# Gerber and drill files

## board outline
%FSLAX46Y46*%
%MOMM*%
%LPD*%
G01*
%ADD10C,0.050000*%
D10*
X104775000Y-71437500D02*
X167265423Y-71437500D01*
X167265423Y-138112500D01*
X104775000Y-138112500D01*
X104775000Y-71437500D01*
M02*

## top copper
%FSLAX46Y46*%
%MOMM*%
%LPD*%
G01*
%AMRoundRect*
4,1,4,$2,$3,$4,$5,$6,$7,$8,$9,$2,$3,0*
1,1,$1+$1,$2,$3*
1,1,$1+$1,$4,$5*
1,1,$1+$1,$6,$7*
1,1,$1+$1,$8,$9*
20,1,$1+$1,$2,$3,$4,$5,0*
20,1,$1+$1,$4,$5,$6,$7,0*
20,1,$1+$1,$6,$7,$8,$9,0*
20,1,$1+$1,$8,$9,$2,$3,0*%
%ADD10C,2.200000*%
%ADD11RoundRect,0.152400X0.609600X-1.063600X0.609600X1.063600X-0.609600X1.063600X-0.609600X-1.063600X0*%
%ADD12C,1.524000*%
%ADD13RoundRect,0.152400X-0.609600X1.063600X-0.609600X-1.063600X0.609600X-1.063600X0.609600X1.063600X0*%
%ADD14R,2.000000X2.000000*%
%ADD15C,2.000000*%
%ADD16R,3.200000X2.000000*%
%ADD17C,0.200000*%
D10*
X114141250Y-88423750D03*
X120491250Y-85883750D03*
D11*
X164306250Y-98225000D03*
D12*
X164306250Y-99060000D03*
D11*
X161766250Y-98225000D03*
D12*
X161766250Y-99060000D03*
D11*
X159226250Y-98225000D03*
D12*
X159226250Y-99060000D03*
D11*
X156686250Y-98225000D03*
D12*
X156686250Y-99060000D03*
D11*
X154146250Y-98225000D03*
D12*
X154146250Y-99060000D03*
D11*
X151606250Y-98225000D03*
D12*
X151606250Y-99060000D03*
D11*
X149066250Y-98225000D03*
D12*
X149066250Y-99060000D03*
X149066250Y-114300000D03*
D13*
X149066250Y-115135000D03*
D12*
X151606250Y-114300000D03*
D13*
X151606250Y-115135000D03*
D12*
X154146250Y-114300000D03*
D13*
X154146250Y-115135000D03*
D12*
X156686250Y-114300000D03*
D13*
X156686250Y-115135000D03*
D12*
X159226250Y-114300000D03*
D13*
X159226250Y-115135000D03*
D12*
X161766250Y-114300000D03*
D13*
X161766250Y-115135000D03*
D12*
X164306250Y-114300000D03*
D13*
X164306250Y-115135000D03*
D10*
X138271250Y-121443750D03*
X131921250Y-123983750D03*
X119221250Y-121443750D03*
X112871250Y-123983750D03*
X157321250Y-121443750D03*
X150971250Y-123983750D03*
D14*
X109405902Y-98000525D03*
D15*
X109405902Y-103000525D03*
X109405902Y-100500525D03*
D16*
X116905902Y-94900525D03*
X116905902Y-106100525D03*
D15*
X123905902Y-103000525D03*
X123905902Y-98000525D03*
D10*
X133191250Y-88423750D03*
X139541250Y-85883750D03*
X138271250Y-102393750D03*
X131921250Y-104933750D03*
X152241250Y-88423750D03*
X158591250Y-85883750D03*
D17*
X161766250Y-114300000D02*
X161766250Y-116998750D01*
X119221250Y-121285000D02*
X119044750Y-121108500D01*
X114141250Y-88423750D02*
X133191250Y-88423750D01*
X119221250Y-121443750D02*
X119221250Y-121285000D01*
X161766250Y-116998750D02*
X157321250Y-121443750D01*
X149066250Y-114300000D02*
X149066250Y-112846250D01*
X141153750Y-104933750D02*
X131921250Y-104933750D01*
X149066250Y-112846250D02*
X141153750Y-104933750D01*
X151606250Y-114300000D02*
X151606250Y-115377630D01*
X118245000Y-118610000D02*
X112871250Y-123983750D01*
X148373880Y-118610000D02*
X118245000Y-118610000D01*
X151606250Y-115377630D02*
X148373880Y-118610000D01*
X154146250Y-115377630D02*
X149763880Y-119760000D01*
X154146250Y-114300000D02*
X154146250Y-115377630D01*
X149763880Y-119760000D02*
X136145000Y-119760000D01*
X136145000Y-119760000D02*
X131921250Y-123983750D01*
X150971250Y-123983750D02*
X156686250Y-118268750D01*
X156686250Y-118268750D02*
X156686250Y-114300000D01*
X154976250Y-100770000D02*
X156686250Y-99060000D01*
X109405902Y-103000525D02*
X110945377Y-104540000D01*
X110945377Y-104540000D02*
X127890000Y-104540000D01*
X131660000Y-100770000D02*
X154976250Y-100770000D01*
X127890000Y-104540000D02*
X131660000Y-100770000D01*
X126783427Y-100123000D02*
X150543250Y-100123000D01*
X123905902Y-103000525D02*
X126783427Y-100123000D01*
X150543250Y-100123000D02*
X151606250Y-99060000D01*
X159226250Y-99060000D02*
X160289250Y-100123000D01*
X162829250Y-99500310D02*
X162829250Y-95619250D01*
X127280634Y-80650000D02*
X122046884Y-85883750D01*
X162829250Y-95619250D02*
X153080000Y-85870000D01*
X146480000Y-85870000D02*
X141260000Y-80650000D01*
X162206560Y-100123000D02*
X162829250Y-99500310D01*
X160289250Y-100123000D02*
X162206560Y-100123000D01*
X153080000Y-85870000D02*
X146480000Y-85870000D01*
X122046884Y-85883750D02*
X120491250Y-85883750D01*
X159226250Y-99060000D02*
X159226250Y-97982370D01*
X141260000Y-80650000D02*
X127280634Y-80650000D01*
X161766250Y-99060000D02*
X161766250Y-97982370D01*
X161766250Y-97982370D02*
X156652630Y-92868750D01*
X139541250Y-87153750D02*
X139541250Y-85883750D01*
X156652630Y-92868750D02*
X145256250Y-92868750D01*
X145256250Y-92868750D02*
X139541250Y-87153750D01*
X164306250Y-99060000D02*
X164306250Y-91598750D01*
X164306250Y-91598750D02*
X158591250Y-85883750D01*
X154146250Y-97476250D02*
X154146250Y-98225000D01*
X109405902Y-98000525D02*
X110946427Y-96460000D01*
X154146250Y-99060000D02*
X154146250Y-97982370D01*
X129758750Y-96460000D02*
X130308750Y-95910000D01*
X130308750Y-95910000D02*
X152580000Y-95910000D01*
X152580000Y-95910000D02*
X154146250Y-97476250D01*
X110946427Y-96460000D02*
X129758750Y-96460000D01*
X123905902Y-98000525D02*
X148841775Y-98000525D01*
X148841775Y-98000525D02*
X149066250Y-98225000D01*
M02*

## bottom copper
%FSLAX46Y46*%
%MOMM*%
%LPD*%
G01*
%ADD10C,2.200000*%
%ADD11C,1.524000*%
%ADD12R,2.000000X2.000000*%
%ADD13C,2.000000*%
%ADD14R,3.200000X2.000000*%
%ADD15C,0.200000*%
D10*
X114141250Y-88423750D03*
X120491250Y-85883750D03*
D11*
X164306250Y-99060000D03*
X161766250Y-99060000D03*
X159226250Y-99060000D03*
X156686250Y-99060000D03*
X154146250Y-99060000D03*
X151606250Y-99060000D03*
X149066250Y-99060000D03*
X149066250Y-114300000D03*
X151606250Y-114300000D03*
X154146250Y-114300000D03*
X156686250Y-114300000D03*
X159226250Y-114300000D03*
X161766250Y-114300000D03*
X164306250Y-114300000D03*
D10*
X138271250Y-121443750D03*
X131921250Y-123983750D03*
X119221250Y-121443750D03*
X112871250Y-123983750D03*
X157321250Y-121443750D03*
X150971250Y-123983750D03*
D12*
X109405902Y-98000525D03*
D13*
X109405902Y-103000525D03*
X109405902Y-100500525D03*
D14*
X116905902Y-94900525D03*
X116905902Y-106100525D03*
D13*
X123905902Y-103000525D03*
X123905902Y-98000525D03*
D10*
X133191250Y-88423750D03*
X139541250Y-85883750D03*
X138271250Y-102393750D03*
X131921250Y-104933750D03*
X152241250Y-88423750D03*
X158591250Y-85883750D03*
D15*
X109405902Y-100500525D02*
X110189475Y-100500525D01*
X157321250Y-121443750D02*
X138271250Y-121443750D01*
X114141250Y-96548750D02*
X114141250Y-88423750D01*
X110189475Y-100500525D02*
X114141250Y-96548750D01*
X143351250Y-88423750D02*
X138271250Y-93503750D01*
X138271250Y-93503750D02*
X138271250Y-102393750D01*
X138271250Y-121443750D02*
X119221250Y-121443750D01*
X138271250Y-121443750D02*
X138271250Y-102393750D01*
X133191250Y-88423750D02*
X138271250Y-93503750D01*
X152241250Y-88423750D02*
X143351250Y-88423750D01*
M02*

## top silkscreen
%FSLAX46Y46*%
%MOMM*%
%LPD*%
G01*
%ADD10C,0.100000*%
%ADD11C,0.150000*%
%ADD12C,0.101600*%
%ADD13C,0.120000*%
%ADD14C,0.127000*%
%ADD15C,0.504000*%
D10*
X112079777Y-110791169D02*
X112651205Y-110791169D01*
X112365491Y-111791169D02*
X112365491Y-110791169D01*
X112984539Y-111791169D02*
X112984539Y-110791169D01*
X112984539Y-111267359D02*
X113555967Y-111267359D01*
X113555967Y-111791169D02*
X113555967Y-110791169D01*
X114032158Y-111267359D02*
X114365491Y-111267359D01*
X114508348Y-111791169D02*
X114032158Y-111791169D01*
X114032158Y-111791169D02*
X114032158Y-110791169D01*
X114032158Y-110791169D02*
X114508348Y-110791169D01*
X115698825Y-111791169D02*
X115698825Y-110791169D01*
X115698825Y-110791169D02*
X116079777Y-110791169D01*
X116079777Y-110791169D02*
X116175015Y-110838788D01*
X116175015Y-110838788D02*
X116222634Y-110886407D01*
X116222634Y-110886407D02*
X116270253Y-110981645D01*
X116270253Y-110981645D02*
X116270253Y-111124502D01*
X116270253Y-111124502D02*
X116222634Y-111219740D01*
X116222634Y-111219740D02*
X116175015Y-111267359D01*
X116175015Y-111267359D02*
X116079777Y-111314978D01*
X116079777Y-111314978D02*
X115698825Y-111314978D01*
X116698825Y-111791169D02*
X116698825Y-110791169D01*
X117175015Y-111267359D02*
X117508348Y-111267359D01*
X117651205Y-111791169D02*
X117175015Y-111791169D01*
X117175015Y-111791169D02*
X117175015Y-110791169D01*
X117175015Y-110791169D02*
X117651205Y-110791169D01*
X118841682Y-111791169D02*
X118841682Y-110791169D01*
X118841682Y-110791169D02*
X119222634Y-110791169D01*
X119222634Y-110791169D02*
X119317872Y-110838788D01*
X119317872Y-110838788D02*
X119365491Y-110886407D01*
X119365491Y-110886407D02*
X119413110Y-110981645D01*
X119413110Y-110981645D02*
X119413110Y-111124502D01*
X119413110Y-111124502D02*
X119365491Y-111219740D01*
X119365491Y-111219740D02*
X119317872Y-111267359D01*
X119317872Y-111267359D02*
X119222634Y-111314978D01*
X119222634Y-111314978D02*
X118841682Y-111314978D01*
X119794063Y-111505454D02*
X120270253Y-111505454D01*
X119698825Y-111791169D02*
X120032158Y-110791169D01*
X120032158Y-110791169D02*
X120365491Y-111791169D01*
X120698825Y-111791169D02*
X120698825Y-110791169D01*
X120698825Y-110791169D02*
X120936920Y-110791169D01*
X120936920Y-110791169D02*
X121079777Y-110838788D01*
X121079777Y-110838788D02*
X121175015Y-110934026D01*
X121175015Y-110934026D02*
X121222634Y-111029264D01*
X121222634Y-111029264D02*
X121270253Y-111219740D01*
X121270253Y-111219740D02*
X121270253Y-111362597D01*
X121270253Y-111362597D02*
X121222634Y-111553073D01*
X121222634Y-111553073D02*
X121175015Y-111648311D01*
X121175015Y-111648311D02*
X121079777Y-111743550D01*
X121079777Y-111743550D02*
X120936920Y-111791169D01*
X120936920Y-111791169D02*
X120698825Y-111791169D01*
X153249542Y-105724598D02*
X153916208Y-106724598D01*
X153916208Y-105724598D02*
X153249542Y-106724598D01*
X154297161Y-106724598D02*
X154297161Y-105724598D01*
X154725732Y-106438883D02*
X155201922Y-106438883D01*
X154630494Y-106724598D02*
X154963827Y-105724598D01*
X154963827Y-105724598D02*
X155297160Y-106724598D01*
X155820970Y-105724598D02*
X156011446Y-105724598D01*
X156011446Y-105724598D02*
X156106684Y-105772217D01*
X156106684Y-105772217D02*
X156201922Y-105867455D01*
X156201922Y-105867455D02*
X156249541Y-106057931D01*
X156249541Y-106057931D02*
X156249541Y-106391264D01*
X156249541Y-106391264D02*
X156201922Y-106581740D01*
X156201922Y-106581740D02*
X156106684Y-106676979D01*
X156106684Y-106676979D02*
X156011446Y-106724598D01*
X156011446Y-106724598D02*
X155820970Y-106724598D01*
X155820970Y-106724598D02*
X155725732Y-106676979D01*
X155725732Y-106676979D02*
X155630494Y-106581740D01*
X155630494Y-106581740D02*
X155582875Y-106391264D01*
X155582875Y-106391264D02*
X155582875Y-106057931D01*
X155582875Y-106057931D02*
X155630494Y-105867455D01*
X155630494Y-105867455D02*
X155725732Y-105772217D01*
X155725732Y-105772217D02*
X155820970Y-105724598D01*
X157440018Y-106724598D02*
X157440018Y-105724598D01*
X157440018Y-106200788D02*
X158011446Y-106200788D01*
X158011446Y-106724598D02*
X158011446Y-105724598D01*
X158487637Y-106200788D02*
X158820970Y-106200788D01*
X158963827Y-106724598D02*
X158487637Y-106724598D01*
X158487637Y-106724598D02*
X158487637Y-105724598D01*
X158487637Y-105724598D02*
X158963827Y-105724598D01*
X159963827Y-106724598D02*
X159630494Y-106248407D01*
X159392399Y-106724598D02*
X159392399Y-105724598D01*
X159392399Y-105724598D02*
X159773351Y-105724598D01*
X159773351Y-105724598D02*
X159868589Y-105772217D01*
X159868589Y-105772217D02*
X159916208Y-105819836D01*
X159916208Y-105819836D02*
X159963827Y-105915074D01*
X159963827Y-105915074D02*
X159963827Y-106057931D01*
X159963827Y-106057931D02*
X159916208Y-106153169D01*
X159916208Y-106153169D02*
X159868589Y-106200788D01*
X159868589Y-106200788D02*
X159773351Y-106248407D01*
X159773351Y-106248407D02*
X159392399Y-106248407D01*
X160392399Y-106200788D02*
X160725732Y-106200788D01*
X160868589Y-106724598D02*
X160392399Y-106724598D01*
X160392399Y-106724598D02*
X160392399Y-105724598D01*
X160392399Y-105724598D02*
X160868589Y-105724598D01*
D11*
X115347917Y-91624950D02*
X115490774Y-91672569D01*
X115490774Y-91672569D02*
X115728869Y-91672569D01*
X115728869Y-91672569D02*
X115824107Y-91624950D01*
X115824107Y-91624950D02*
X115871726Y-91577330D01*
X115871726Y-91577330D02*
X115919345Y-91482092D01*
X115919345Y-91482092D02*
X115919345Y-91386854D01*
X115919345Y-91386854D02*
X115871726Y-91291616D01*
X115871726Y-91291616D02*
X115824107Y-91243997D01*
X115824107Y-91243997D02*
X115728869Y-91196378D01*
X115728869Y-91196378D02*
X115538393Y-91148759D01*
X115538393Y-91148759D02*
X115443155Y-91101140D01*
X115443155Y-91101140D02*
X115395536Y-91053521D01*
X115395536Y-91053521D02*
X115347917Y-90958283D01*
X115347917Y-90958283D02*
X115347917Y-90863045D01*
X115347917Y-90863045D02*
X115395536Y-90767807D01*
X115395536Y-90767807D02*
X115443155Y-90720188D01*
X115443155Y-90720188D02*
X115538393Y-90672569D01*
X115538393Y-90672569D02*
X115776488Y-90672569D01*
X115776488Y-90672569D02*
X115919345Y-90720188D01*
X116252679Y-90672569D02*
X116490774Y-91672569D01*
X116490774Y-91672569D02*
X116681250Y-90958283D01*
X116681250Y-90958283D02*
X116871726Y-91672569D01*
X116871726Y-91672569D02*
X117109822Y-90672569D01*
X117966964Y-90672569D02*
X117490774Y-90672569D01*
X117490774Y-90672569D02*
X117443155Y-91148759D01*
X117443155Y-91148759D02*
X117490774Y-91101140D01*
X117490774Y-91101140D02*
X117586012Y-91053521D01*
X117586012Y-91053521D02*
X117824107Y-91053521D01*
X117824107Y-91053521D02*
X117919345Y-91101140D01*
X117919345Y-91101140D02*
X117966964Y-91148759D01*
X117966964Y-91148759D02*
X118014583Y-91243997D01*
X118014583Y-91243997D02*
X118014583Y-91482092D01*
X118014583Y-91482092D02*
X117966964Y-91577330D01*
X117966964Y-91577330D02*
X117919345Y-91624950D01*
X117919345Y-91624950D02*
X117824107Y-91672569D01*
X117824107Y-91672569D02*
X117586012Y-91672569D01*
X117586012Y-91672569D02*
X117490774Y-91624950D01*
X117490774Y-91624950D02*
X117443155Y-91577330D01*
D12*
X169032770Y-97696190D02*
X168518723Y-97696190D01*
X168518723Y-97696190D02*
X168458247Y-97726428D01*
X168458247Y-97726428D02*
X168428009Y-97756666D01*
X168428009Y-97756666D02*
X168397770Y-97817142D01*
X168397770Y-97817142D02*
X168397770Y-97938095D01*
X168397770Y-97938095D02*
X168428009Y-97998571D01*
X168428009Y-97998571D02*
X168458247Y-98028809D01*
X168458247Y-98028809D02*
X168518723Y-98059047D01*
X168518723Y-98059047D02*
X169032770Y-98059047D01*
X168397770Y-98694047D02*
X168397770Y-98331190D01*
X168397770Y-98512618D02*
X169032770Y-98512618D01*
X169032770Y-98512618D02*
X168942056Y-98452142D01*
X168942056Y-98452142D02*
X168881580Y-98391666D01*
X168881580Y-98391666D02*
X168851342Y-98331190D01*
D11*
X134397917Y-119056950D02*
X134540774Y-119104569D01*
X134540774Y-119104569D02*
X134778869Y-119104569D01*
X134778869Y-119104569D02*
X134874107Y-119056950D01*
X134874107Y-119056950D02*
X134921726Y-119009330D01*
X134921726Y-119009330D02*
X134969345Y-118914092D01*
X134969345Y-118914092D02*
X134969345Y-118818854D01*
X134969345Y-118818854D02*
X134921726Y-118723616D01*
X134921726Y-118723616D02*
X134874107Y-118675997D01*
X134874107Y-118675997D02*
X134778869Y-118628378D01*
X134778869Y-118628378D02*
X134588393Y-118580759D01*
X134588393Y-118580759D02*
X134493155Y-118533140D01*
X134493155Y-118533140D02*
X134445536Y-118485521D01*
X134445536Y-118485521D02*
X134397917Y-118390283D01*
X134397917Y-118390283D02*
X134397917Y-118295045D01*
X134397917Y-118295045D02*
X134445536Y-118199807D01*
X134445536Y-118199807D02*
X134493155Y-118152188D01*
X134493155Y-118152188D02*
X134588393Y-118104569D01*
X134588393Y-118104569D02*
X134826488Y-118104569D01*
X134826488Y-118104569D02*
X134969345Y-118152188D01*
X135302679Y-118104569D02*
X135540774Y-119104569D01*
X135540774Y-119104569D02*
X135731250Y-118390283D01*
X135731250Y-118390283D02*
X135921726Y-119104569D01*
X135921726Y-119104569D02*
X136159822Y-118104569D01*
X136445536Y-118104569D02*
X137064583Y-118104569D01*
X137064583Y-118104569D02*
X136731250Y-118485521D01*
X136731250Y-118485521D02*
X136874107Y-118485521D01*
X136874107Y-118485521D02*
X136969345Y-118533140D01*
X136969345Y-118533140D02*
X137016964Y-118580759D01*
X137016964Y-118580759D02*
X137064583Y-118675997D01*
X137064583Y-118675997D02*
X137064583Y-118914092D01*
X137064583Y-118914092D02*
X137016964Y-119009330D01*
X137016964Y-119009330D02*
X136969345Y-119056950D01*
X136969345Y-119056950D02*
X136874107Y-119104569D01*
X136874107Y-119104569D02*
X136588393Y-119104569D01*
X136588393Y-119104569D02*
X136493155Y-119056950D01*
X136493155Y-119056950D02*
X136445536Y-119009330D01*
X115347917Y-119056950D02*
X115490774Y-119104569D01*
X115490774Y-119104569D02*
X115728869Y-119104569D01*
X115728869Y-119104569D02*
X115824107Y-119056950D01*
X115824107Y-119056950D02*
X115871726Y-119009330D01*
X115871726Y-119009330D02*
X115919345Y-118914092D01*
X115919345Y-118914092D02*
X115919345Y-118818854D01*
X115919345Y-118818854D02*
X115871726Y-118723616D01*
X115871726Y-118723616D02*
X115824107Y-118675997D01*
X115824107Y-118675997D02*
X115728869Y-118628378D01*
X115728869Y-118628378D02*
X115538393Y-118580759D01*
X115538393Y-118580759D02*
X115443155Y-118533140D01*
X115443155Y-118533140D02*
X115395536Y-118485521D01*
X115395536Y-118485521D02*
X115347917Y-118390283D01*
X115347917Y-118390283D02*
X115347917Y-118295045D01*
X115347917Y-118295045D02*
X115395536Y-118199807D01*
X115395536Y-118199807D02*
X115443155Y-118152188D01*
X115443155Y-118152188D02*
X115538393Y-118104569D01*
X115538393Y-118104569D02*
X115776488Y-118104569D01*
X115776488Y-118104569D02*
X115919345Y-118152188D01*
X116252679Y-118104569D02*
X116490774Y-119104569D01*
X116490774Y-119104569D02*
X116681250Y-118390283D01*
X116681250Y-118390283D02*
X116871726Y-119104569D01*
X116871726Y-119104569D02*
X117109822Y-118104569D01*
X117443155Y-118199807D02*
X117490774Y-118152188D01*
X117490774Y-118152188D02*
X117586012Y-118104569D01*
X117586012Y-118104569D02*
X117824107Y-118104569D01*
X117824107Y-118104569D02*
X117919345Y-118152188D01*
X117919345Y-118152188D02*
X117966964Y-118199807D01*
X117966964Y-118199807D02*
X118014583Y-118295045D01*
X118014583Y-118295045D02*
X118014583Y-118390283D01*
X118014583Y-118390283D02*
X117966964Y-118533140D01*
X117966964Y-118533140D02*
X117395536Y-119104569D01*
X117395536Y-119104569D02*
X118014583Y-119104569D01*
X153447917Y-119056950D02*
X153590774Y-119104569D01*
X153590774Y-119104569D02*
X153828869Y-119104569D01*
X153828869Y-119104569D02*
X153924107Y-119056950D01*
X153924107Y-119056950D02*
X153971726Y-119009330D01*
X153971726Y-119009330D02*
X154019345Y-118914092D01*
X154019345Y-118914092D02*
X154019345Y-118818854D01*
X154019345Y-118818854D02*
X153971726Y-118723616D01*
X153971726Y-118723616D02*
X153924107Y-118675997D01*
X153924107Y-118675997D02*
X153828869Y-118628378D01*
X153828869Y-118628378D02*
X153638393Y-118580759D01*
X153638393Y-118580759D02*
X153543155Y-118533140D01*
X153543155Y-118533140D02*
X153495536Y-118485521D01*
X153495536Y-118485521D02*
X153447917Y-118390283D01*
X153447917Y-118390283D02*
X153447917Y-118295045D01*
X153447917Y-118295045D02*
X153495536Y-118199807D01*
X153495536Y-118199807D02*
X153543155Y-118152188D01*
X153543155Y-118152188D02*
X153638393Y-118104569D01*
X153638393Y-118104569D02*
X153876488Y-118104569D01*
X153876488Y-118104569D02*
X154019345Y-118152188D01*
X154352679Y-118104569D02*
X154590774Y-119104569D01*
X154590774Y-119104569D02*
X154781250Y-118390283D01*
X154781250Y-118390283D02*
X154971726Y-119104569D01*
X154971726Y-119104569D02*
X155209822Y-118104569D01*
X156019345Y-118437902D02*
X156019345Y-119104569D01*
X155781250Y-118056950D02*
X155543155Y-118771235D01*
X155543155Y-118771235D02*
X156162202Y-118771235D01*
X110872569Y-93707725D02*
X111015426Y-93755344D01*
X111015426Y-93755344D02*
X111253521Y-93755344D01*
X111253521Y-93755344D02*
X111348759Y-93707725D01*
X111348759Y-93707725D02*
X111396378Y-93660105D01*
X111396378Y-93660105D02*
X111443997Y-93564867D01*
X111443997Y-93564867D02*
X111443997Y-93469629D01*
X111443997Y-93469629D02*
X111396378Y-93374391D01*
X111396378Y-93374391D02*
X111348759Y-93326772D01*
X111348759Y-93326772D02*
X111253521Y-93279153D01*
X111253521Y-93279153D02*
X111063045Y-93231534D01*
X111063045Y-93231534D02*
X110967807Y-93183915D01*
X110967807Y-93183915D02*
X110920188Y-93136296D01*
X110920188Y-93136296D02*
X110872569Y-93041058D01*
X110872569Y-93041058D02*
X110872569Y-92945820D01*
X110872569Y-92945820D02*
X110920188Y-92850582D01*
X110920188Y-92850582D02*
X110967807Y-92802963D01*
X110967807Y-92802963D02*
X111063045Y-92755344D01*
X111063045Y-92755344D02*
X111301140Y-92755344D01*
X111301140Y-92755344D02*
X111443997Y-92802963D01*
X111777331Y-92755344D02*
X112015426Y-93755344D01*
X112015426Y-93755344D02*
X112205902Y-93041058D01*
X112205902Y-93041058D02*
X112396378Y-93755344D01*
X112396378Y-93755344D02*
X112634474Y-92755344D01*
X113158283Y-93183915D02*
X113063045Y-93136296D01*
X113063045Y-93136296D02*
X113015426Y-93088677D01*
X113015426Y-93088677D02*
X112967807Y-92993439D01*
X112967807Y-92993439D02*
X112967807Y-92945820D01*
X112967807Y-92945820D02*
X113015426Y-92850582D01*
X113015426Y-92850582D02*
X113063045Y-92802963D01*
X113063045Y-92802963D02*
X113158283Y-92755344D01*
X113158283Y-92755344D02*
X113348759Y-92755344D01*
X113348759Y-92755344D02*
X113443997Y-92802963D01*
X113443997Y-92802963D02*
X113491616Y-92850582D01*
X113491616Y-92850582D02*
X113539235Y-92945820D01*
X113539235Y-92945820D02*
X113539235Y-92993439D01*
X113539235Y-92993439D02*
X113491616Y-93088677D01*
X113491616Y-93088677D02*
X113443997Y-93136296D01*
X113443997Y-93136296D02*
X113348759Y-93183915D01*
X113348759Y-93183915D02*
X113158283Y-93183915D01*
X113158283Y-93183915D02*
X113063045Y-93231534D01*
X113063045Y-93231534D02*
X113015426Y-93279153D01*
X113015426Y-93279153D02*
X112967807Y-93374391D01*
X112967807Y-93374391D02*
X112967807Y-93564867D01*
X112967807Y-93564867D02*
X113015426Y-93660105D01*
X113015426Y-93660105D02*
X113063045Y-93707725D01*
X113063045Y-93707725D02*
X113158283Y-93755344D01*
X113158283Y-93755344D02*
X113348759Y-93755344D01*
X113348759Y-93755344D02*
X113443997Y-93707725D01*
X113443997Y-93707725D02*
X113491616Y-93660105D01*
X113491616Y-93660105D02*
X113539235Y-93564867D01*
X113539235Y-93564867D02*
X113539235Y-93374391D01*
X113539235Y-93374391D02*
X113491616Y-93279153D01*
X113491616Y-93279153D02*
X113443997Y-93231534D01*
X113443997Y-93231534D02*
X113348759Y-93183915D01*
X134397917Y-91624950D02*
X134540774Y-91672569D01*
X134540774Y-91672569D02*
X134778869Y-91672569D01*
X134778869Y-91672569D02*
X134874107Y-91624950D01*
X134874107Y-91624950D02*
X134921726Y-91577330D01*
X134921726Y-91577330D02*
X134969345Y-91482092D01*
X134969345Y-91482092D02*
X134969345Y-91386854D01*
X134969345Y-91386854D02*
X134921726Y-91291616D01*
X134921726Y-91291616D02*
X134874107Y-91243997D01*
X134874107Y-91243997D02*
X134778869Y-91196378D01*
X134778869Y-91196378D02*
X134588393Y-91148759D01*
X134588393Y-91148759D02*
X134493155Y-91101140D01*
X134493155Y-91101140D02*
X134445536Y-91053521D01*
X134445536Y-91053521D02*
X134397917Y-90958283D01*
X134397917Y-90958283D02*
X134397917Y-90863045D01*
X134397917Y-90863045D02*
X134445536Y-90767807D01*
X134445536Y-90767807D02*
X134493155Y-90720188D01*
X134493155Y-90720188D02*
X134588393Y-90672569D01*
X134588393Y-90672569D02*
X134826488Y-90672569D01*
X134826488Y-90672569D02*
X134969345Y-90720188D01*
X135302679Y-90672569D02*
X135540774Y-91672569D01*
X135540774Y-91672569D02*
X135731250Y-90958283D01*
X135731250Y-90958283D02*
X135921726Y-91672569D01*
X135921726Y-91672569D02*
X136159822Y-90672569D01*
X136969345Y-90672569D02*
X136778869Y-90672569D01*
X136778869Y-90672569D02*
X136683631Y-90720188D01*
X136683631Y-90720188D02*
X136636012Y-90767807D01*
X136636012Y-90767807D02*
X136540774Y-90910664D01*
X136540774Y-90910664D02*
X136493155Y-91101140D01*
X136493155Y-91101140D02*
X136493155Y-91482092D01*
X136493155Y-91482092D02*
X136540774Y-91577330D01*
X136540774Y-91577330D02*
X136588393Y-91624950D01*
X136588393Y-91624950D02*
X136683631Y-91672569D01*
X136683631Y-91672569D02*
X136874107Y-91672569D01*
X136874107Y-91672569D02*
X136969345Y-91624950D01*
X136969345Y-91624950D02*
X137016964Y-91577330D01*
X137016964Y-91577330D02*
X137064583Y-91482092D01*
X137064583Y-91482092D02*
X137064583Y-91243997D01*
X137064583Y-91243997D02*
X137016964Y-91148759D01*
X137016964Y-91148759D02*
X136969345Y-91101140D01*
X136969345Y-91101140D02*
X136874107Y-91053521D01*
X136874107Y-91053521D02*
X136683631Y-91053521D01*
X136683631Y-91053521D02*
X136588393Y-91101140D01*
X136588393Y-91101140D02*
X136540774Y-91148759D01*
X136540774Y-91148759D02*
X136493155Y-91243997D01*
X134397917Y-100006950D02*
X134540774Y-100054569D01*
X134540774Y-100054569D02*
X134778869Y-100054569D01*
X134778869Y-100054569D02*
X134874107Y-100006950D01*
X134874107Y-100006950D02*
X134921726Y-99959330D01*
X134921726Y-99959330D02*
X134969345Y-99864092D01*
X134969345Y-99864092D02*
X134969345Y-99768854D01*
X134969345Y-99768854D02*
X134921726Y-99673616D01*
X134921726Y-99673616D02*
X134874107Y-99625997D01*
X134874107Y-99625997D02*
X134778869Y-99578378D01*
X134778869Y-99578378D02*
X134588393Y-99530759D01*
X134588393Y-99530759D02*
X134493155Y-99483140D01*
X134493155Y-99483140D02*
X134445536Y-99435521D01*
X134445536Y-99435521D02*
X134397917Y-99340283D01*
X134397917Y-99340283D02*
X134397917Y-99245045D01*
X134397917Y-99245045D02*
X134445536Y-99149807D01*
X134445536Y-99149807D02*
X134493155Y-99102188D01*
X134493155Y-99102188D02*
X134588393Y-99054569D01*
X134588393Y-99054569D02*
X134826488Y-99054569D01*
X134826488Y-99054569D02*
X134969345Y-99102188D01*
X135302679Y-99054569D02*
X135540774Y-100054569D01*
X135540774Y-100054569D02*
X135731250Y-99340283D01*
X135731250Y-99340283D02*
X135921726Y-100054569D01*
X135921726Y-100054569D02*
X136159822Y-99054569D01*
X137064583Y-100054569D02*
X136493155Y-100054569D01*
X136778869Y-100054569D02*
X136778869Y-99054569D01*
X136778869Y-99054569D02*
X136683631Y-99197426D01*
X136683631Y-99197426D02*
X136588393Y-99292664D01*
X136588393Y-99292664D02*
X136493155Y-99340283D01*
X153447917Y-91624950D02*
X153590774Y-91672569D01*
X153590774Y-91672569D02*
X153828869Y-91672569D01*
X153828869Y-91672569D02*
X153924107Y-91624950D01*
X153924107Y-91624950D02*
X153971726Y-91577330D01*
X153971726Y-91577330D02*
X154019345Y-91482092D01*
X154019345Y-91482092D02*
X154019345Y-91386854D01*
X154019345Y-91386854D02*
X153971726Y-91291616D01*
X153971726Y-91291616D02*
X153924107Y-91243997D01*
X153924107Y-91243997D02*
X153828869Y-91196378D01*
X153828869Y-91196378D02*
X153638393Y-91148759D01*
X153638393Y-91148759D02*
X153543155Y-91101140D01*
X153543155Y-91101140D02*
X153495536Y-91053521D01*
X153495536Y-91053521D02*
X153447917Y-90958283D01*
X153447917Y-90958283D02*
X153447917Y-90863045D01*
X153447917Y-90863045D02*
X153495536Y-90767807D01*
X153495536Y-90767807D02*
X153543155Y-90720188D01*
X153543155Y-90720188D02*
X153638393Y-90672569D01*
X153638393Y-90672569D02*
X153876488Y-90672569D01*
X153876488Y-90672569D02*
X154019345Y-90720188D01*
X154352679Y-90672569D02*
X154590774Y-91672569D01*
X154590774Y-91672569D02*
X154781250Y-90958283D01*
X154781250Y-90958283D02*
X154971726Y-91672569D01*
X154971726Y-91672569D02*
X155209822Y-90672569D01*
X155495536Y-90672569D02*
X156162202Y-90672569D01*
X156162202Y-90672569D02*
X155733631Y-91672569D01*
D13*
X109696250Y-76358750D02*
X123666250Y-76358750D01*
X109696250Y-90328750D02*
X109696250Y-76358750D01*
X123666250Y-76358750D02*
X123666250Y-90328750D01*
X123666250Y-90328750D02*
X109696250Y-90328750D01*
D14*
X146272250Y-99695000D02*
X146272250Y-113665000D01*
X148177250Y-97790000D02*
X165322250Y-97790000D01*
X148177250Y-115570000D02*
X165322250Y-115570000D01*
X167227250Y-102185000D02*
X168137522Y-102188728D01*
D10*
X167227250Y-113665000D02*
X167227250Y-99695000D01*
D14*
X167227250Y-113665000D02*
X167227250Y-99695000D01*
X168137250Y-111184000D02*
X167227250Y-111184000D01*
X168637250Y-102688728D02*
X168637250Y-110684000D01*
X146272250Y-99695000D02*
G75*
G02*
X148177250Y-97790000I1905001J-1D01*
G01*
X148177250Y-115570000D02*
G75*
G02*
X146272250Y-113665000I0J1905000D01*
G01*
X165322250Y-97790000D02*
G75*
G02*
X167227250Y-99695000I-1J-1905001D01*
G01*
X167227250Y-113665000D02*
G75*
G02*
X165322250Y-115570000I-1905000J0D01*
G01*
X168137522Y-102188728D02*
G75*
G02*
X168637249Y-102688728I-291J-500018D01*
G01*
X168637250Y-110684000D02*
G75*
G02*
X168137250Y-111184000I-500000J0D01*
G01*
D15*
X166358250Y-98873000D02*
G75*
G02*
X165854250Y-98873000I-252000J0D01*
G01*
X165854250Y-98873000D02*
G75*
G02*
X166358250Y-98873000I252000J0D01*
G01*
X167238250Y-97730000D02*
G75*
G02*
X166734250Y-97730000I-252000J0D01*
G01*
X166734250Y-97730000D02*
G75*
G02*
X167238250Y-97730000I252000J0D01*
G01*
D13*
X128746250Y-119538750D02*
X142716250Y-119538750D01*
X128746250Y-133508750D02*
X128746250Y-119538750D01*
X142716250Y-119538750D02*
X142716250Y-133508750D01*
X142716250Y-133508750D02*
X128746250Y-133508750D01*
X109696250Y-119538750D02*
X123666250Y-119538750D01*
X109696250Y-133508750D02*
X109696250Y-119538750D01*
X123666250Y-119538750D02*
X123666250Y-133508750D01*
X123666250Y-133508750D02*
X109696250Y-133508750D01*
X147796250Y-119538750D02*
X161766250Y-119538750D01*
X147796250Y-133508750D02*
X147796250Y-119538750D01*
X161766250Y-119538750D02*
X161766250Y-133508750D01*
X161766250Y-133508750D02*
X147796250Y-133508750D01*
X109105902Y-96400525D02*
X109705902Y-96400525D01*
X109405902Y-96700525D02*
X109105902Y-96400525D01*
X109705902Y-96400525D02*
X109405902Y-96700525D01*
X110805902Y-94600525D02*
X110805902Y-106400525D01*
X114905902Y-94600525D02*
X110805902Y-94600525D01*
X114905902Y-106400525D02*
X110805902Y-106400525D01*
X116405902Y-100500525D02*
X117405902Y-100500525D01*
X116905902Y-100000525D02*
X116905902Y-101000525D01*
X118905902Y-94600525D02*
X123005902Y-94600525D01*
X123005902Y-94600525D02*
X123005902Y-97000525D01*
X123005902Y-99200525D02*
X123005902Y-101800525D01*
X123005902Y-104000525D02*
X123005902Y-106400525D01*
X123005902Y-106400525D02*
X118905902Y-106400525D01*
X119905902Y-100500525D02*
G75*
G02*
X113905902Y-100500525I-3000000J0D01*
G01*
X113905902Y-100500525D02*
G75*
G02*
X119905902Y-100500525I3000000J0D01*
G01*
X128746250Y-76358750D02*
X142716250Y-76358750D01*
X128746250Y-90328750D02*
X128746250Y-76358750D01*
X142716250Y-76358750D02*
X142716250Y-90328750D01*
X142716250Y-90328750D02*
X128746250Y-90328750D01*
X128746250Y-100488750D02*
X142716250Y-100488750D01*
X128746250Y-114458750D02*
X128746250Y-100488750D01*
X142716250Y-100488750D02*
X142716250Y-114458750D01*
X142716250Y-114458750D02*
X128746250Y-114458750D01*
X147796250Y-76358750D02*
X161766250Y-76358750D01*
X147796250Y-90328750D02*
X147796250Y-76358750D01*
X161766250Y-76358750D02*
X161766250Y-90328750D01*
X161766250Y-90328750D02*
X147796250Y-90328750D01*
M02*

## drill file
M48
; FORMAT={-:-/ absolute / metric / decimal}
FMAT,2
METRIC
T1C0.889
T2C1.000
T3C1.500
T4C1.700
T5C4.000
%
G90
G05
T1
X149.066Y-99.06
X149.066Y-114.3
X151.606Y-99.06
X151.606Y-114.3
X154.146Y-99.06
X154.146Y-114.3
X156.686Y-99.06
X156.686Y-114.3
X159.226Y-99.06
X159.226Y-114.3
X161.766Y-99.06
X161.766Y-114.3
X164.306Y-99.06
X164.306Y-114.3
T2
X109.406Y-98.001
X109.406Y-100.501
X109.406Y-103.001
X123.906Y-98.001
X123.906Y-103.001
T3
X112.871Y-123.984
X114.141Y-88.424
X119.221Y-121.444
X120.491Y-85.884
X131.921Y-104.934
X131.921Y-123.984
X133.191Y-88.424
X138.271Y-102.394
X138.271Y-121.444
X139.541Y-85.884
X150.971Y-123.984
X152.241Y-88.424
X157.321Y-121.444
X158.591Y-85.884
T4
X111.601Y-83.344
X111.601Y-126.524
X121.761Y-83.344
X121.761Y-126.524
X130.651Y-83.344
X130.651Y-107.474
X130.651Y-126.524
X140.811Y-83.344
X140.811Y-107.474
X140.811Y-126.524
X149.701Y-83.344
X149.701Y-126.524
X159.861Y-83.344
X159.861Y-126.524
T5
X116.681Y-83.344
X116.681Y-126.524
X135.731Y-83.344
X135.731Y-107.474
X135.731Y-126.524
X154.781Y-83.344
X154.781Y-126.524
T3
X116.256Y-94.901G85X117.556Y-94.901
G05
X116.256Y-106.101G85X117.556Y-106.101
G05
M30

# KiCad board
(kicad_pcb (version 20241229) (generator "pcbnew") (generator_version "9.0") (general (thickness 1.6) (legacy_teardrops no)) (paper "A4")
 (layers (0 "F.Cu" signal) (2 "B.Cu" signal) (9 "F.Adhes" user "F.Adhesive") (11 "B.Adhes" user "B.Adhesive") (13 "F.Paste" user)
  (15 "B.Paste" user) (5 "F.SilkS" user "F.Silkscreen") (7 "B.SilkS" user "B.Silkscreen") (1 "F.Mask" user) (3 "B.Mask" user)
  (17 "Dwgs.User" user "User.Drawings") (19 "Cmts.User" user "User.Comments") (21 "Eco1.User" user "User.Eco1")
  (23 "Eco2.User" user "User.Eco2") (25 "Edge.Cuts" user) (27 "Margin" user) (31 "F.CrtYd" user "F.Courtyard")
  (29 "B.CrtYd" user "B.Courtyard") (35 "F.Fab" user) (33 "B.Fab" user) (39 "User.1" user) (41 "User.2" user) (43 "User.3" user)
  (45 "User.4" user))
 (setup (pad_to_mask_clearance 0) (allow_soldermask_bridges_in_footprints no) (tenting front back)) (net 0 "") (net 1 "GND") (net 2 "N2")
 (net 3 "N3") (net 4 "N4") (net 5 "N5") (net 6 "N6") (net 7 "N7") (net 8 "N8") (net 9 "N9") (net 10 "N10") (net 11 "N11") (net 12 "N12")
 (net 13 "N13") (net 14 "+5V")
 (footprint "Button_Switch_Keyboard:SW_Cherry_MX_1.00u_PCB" (layer "F.Cu") (at 114.14125 88.42375 180)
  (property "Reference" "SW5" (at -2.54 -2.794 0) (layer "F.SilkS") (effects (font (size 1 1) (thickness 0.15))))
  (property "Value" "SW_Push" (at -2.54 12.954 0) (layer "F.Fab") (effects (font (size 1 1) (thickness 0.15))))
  (fp_line (start 4.445 12.065) (end -9.525 12.065) (stroke (width 0.12) (type solid)) (layer "F.SilkS"))
  (fp_line (start 4.445 -1.905) (end 4.445 12.065) (stroke (width 0.12) (type solid)) (layer "F.SilkS"))
  (fp_line (start -9.525 12.065) (end -9.525 -1.905) (stroke (width 0.12) (type solid)) (layer "F.SilkS"))
  (fp_line (start -9.525 -1.905) (end 4.445 -1.905) (stroke (width 0.12) (type solid)) (layer "F.SilkS"))
  (pad "" np_thru_hole circle (at -7.62 5.08 180) (size 1.7 1.7) (drill 1.7) (layers "*.Cu" "*.Mask"))
  (pad "" np_thru_hole circle (at -2.54 5.08 180) (size 4 4) (drill 4) (layers "*.Cu" "*.Mask"))
  (pad "" np_thru_hole circle (at 2.54 5.08 180) (size 1.7 1.7) (drill 1.7) (layers "*.Cu" "*.Mask"))
  (pad "1" thru_hole circle (at 0 0 180) (size 2.2 2.2) (drill 1.5) (layers "*.Cu" "*.Mask") (remove_unused_layers no) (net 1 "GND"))
  (pad "2" thru_hole circle (at -6.35 2.54 180) (size 2.2 2.2) (drill 1.5) (layers "*.Cu" "*.Mask") (remove_unused_layers no) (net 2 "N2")))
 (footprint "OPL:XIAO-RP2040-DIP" (layer "F.Cu") (at 156.68625 106.68 -90)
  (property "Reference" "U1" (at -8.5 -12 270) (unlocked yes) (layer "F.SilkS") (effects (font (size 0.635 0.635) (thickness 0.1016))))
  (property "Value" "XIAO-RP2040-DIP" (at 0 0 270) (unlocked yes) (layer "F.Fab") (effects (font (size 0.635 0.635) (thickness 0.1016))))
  (fp_line (start -6.985 10.414) (end 6.985 10.414) (stroke (width 0.127) (type solid)) (layer "F.SilkS"))
  (fp_line (start -8.89 8.509) (end -8.89 -8.636) (stroke (width 0.127) (type solid)) (layer "F.SilkS"))
  (fp_line (start 8.89 8.509) (end 8.89 -8.636) (stroke (width 0.127) (type solid)) (layer "F.SilkS"))
  (fp_line (start -4.495 -10.541) (end -4.491272 -11.451272) (stroke (width 0.127) (type solid)) (layer "F.SilkS"))
  (fp_line (start 6.985 -10.541) (end -6.985 -10.541) (stroke (width 0.1) (type solid)) (layer "F.SilkS"))
  (fp_line (start 6.985 -10.541) (end -6.985 -10.541) (stroke (width 0.127) (type solid)) (layer "F.SilkS"))
  (fp_line (start 4.504 -11.451) (end 4.504 -10.541) (stroke (width 0.127) (type solid)) (layer "F.SilkS"))
  (fp_line (start -3.991272 -11.951) (end 4.004 -11.951) (stroke (width 0.127) (type solid)) (layer "F.SilkS"))
  (fp_arc (start -6.985 10.414) (mid -8.332038 9.856038) (end -8.89 8.509) (stroke (width 0.127) (type solid)) (layer "F.SilkS"))
  (fp_arc (start 8.89 8.509) (mid 8.332038 9.856038) (end 6.985 10.414) (stroke (width 0.127) (type solid)) (layer "F.SilkS"))
  (fp_arc (start -8.89 -8.636) (mid -8.332038 -9.983038) (end -6.985 -10.541) (stroke (width 0.127) (type solid)) (layer "F.SilkS"))
  (fp_arc (start 6.985 -10.541) (mid 8.332038 -9.983038) (end 8.89 -8.636) (stroke (width 0.127) (type solid)) (layer "F.SilkS"))
  (fp_arc (start -4.491272 -11.451272) (mid -4.344728 -11.80464) (end -3.991272 -11.951) (stroke (width 0.127) (type default))
   (layer "F.SilkS"))
  (fp_arc (start 4.004 -11.951) (mid 4.357553 -11.804553) (end 4.504 -11.451) (stroke (width 0.127) (type default)) (layer "F.SilkS"))
  (fp_circle (center -7.807 -9.42) (end -7.807 -9.674) (stroke (width 0.5) (type solid)) (fill yes) (layer "F.SilkS"))
  (fp_circle (center -8.95 -10.3) (end -8.95 -10.554) (stroke (width 0.5) (type solid)) (fill yes) (layer "F.SilkS"))
  (pad "1" smd roundrect (at -8.455 -7.62 90) (size 2.432 1.524) (layers "F.Cu" "F.Mask") (roundrect_rratio 0.1) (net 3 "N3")
   (thermal_bridge_angle 45))
  (pad "1" thru_hole circle (at -7.62 -7.62 90) (size 1.524 1.524) (drill 0.889) (layers "*.Cu" "*.Mask") (remove_unused_layers no)
   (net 3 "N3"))
  (pad "2" smd roundrect (at -8.455 -5.08 90) (size 2.432 1.524) (layers "F.Cu" "F.Mask") (roundrect_rratio 0.1) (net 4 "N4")
   (thermal_bridge_angle 45))
  (pad "2" thru_hole circle (at -7.62 -5.08 90) (size 1.524 1.524) (drill 0.889) (layers "*.Cu" "*.Mask") (remove_unused_layers no)
   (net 4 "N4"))
  (pad "3" smd roundrect (at -8.455 -2.54 90) (size 2.432 1.524) (layers "F.Cu" "F.Mask") (roundrect_rratio 0.1) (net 2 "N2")
   (thermal_bridge_angle 45))
  (pad "3" thru_hole circle (at -7.62 -2.54 90) (size 1.524 1.524) (drill 0.889) (layers "*.Cu" "*.Mask") (remove_unused_layers no)
   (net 2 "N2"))
  (pad "4" smd roundrect (at -8.455 0 90) (size 2.432 1.524) (layers "F.Cu" "F.Mask") (roundrect_rratio 0.1) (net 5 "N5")
   (thermal_bridge_angle 45))
  (pad "4" thru_hole circle (at -7.62 0 90) (size 1.524 1.524) (drill 0.889) (layers "*.Cu" "*.Mask") (remove_unused_layers no) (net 5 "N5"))
  (pad "5" smd roundrect (at -8.455 2.54 90) (size 2.432 1.524) (layers "F.Cu" "F.Mask") (roundrect_rratio 0.1) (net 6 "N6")
   (thermal_bridge_angle 45))
  (pad "5" thru_hole circle (at -7.62 2.54 90) (size 1.524 1.524) (drill 0.889) (layers "*.Cu" "*.Mask") (remove_unused_layers no)
   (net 6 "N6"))
  (pad "6" smd roundrect (at -8.455 5.08 90) (size 2.432 1.524) (layers "F.Cu" "F.Mask") (roundrect_rratio 0.1) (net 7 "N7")
   (thermal_bridge_angle 45))
  (pad "6" thru_hole circle (at -7.62 5.08 90) (size 1.524 1.524) (drill 0.889) (layers "*.Cu" "*.Mask") (remove_unused_layers no)
   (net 7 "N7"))
  (pad "7" smd roundrect (at -8.455 7.62 90) (size 2.432 1.524) (layers "F.Cu" "F.Mask") (roundrect_rratio 0.1) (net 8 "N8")
   (thermal_bridge_angle 45))
  (pad "7" thru_hole circle (at -7.62 7.62 90) (size 1.524 1.524) (drill 0.889) (layers "*.Cu" "*.Mask") (remove_unused_layers no)
   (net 8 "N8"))
  (pad "8" thru_hole circle (at 7.62 7.62 270) (size 1.524 1.524) (drill 0.889) (layers "*.Cu" "*.Mask") (remove_unused_layers no)
   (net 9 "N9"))
  (pad "8" smd roundrect (at 8.455 7.62 270) (size 2.432 1.524) (layers "F.Cu" "F.Mask") (roundrect_rratio 0.1) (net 9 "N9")
   (thermal_bridge_angle 45))
  (pad "9" thru_hole circle (at 7.62 5.08 270) (size 1.524 1.524) (drill 0.889) (layers "*.Cu" "*.Mask") (remove_unused_layers no)
   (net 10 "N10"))
  (pad "9" smd roundrect (at 8.455 5.08 270) (size 2.432 1.524) (layers "F.Cu" "F.Mask") (roundrect_rratio 0.1) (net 10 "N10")
   (thermal_bridge_angle 45))
  (pad "10" thru_hole circle (at 7.62 2.54 270) (size 1.524 1.524) (drill 0.889) (layers "*.Cu" "*.Mask") (remove_unused_layers no)
   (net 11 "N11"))
  (pad "10" smd roundrect (at 8.455 2.54 270) (size 2.432 1.524) (layers "F.Cu" "F.Mask") (roundrect_rratio 0.1) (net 11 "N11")
   (thermal_bridge_angle 45))
  (pad "11" thru_hole circle (at 7.62 0 270) (size 1.524 1.524) (drill 0.889) (layers "*.Cu" "*.Mask") (remove_unused_layers no)
   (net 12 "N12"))
  (pad "11" smd roundrect (at 8.455 0 270) (size 2.432 1.524) (layers "F.Cu" "F.Mask") (roundrect_rratio 0.1) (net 12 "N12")
   (thermal_bridge_angle 45))
  (pad "12" thru_hole circle (at 7.62 -2.54 270) (size 1.524 1.524) (drill 0.889) (layers "*.Cu" "*.Mask") (remove_unused_layers no)
   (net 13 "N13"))
  (pad "12" smd roundrect (at 8.455 -2.54 270) (size 2.432 1.524) (layers "F.Cu" "F.Mask") (roundrect_rratio 0.1) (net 13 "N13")
   (thermal_bridge_angle 45))
  (pad "13" thru_hole circle (at 7.62 -5.08 270) (size 1.524 1.524) (drill 0.889) (layers "*.Cu" "*.Mask") (remove_unused_layers no)
   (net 1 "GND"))
  (pad "13" smd roundrect (at 8.455 -5.08 270) (size 2.432 1.524) (layers "F.Cu" "F.Mask") (roundrect_rratio 0.1) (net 1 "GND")
   (thermal_bridge_angle 45))
  (pad "14" thru_hole circle (at 7.62 -7.62 270) (size 1.524 1.524) (drill 0.889) (layers "*.Cu" "*.Mask") (remove_unused_layers no)
   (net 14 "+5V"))
  (pad "14" smd roundrect (at 8.455 -7.62 270) (size 2.432 1.524) (layers "F.Cu" "F.Mask") (roundrect_rratio 0.1) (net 14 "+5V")
   (thermal_bridge_angle 45)))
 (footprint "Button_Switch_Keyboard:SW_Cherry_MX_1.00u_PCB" (layer "F.Cu") (at 138.27125 121.44375)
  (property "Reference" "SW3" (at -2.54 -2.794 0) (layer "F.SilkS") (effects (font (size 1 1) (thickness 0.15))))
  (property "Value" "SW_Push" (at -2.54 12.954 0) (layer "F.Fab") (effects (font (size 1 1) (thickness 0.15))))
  (fp_line (start -9.525 -1.905) (end 4.445 -1.905) (stroke (width 0.12) (type solid)) (layer "F.SilkS"))
  (fp_line (start -9.525 12.065) (end -9.525 -1.905) (stroke (width 0.12) (type solid)) (layer "F.SilkS"))
  (fp_line (start 4.445 -1.905) (end 4.445 12.065) (stroke (width 0.12) (type solid)) (layer "F.SilkS"))
  (fp_line (start 4.445 12.065) (end -9.525 12.065) (stroke (width 0.12) (type solid)) (layer "F.SilkS"))
  (pad "" np_thru_hole circle (at -7.62 5.08) (size 1.7 1.7) (drill 1.7) (layers "*.Cu" "*.Mask"))
  (pad "" np_thru_hole circle (at -2.54 5.08) (size 4 4) (drill 4) (layers "*.Cu" "*.Mask"))
  (pad "" np_thru_hole circle (at 2.54 5.08) (size 1.7 1.7) (drill 1.7) (layers "*.Cu" "*.Mask"))
  (pad "1" thru_hole circle (at 0 0) (size 2.2 2.2) (drill 1.5) (layers "*.Cu" "*.Mask") (remove_unused_layers no) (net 1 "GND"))
  (pad "2" thru_hole circle (at -6.35 2.54) (size 2.2 2.2) (drill 1.5) (layers "*.Cu" "*.Mask") (remove_unused_layers no) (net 11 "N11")))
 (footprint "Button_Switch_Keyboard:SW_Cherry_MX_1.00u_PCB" (layer "F.Cu") (at 119.22125 121.44375)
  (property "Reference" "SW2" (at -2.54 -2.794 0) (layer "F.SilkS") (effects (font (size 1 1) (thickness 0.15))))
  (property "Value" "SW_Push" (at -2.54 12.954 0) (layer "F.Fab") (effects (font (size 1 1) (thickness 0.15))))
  (fp_line (start -9.525 -1.905) (end 4.445 -1.905) (stroke (width 0.12) (type solid)) (layer "F.SilkS"))
  (fp_line (start -9.525 12.065) (end -9.525 -1.905) (stroke (width 0.12) (type solid)) (layer "F.SilkS"))
  (fp_line (start 4.445 -1.905) (end 4.445 12.065) (stroke (width 0.12) (type solid)) (layer "F.SilkS"))
  (fp_line (start 4.445 12.065) (end -9.525 12.065) (stroke (width 0.12) (type solid)) (layer "F.SilkS"))
  (pad "" np_thru_hole circle (at -7.62 5.08) (size 1.7 1.7) (drill 1.7) (layers "*.Cu" "*.Mask"))
  (pad "" np_thru_hole circle (at -2.54 5.08) (size 4 4) (drill 4) (layers "*.Cu" "*.Mask"))
  (pad "" np_thru_hole circle (at 2.54 5.08) (size 1.7 1.7) (drill 1.7) (layers "*.Cu" "*.Mask"))
  (pad "1" thru_hole circle (at 0 0) (size 2.2 2.2) (drill 1.5) (layers "*.Cu" "*.Mask") (remove_unused_layers no) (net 1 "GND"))
  (pad "2" thru_hole circle (at -6.35 2.54) (size 2.2 2.2) (drill 1.5) (layers "*.Cu" "*.Mask") (remove_unused_layers no) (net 10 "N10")))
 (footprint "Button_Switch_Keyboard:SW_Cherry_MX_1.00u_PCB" (layer "F.Cu") (at 157.32125 121.44375)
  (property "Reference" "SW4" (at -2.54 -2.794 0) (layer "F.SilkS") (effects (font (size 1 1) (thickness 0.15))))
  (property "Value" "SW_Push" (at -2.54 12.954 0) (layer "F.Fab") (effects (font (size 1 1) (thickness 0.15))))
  (fp_line (start -9.525 -1.905) (end 4.445 -1.905) (stroke (width 0.12) (type solid)) (layer "F.SilkS"))
  (fp_line (start -9.525 12.065) (end -9.525 -1.905) (stroke (width 0.12) (type solid)) (layer "F.SilkS"))
  (fp_line (start 4.445 -1.905) (end 4.445 12.065) (stroke (width 0.12) (type solid)) (layer "F.SilkS"))
  (fp_line (start 4.445 12.065) (end -9.525 12.065) (stroke (width 0.12) (type solid)) (layer "F.SilkS"))
  (pad "" np_thru_hole circle (at -7.62 5.08) (size 1.7 1.7) (drill 1.7) (layers "*.Cu" "*.Mask"))
  (pad "" np_thru_hole circle (at -2.54 5.08) (size 4 4) (drill 4) (layers "*.Cu" "*.Mask"))
  (pad "" np_thru_hole circle (at 2.54 5.08) (size 1.7 1.7) (drill 1.7) (layers "*.Cu" "*.Mask"))
  (pad "1" thru_hole circle (at 0 0) (size 2.2 2.2) (drill 1.5) (layers "*.Cu" "*.Mask") (remove_unused_layers no) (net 1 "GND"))
  (pad "2" thru_hole circle (at -6.35 2.54) (size 2.2 2.2) (drill 1.5) (layers "*.Cu" "*.Mask") (remove_unused_layers no) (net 12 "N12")))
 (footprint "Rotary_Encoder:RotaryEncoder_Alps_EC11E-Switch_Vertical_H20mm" (layer "F.Cu") (at 109.405902 98.000525)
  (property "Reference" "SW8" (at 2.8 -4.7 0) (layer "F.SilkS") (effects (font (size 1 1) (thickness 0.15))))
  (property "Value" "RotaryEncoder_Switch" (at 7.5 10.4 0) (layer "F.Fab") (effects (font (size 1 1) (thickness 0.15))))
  (fp_line (start -0.3 -1.6) (end 0.3 -1.6) (stroke (width 0.12) (type solid)) (layer "F.SilkS"))
  (fp_line (start 0 -1.3) (end -0.3 -1.6) (stroke (width 0.12) (type solid)) (layer "F.SilkS"))
  (fp_line (start 0.3 -1.6) (end 0 -1.3) (stroke (width 0.12) (type solid)) (layer "F.SilkS"))
  (fp_line (start 1.4 -3.4) (end 1.4 8.4) (stroke (width 0.12) (type solid)) (layer "F.SilkS"))
  (fp_line (start 5.5 -3.4) (end 1.4 -3.4) (stroke (width 0.12) (type solid)) (layer "F.SilkS"))
  (fp_line (start 5.5 8.4) (end 1.4 8.4) (stroke (width 0.12) (type solid)) (layer "F.SilkS"))
  (fp_line (start 7 2.5) (end 8 2.5) (stroke (width 0.12) (type solid)) (layer "F.SilkS"))
  (fp_line (start 7.5 2) (end 7.5 3) (stroke (width 0.12) (type solid)) (layer "F.SilkS"))
  (fp_line (start 9.5 -3.4) (end 13.6 -3.4) (stroke (width 0.12) (type solid)) (layer "F.SilkS"))
  (fp_line (start 13.6 -3.4) (end 13.6 -1) (stroke (width 0.12) (type solid)) (layer "F.SilkS"))
  (fp_line (start 13.6 1.2) (end 13.6 3.8) (stroke (width 0.12) (type solid)) (layer "F.SilkS"))
  (fp_line (start 13.6 6) (end 13.6 8.4) (stroke (width 0.12) (type solid)) (layer "F.SilkS"))
  (fp_line (start 13.6 8.4) (end 9.5 8.4) (stroke (width 0.12) (type solid)) (layer "F.SilkS"))
  (fp_circle (center 7.5 2.5) (end 10.5 2.5) (stroke (width 0.12) (type solid)) (fill no) (layer "F.SilkS"))
  (pad "A" thru_hole rect (at 0 0) (size 2 2) (drill 1) (layers "*.Cu" "*.Mask") (remove_unused_layers no) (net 6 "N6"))
  (pad "B" thru_hole circle (at 0 5) (size 2 2) (drill 1) (layers "*.Cu" "*.Mask") (remove_unused_layers no) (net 5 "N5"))
  (pad "C" thru_hole circle (at 0 2.5) (size 2 2) (drill 1) (layers "*.Cu" "*.Mask") (remove_unused_layers no) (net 1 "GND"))
  (pad "MP" thru_hole rect (at 7.5 -3.1) (size 3.2 2) (drill oval 2.8 1.5) (layers "*.Cu" "*.Mask") (remove_unused_layers no))
  (pad "MP" thru_hole rect (at 7.5 8.1) (size 3.2 2) (drill oval 2.8 1.5) (layers "*.Cu" "*.Mask") (remove_unused_layers no))
  (pad "S1" thru_hole circle (at 14.5 5) (size 2 2) (drill 1) (layers "*.Cu" "*.Mask") (remove_unused_layers no) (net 7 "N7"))
  (pad "S2" thru_hole circle (at 14.5 0) (size 2 2) (drill 1) (layers "*.Cu" "*.Mask") (remove_unused_layers no) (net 8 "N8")))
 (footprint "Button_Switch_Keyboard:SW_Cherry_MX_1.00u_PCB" (layer "F.Cu") (at 133.19125 88.42375 180)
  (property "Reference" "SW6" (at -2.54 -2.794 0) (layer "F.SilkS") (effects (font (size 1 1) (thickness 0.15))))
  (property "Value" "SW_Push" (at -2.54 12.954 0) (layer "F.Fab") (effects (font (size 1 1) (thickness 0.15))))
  (fp_line (start 4.445 12.065) (end -9.525 12.065) (stroke (width 0.12) (type solid)) (layer "F.SilkS"))
  (fp_line (start 4.445 -1.905) (end 4.445 12.065) (stroke (width 0.12) (type solid)) (layer "F.SilkS"))
  (fp_line (start -9.525 12.065) (end -9.525 -1.905) (stroke (width 0.12) (type solid)) (layer "F.SilkS"))
  (fp_line (start -9.525 -1.905) (end 4.445 -1.905) (stroke (width 0.12) (type solid)) (layer "F.SilkS"))
  (pad "" np_thru_hole circle (at -7.62 5.08 180) (size 1.7 1.7) (drill 1.7) (layers "*.Cu" "*.Mask"))
  (pad "" np_thru_hole circle (at -2.54 5.08 180) (size 4 4) (drill 4) (layers "*.Cu" "*.Mask"))
  (pad "" np_thru_hole circle (at 2.54 5.08 180) (size 1.7 1.7) (drill 1.7) (layers "*.Cu" "*.Mask"))
  (pad "1" thru_hole circle (at 0 0 180) (size 2.2 2.2) (drill 1.5) (layers "*.Cu" "*.Mask") (remove_unused_layers no) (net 1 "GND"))
  (pad "2" thru_hole circle (at -6.35 2.54 180) (size 2.2 2.2) (drill 1.5) (layers "*.Cu" "*.Mask") (remove_unused_layers no) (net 4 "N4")))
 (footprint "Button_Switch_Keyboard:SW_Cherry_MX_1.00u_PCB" (layer "F.Cu") (at 138.27125 102.39375)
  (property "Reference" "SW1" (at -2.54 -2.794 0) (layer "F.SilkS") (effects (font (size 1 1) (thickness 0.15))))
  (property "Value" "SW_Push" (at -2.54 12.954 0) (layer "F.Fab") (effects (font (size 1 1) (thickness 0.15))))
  (fp_line (start -9.525 -1.905) (end 4.445 -1.905) (stroke (width 0.12) (type solid)) (layer "F.SilkS"))
  (fp_line (start -9.525 12.065) (end -9.525 -1.905) (stroke (width 0.12) (type solid)) (layer "F.SilkS"))
  (fp_line (start 4.445 -1.905) (end 4.445 12.065) (stroke (width 0.12) (type solid)) (layer "F.SilkS"))
  (fp_line (start 4.445 12.065) (end -9.525 12.065) (stroke (width 0.12) (type solid)) (layer "F.SilkS"))
  (pad "" np_thru_hole circle (at -7.62 5.08) (size 1.7 1.7) (drill 1.7) (layers "*.Cu" "*.Mask"))
  (pad "" np_thru_hole circle (at -2.54 5.08) (size 4 4) (drill 4) (layers "*.Cu" "*.Mask"))
  (pad "" np_thru_hole circle (at 2.54 5.08) (size 1.7 1.7) (drill 1.7) (layers "*.Cu" "*.Mask"))
  (pad "1" thru_hole circle (at 0 0) (size 2.2 2.2) (drill 1.5) (layers "*.Cu" "*.Mask") (remove_unused_layers no) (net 1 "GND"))
  (pad "2" thru_hole circle (at -6.35 2.54) (size 2.2 2.2) (drill 1.5) (layers "*.Cu" "*.Mask") (remove_unused_layers no) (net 9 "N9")))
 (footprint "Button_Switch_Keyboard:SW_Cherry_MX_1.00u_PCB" (layer "F.Cu") (at 152.24125 88.42375 180)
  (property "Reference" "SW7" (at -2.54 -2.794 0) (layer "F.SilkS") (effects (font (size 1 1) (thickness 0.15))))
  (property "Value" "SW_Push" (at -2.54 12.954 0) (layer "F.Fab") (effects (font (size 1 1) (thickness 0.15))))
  (fp_line (start 4.445 12.065) (end -9.525 12.065) (stroke (width 0.12) (type solid)) (layer "F.SilkS"))
  (fp_line (start 4.445 -1.905) (end 4.445 12.065) (stroke (width 0.12) (type solid)) (layer "F.SilkS"))
  (fp_line (start -9.525 12.065) (end -9.525 -1.905) (stroke (width 0.12) (type solid)) (layer "F.SilkS"))
  (fp_line (start -9.525 -1.905) (end 4.445 -1.905) (stroke (width 0.12) (type solid)) (layer "F.SilkS"))
  (pad "" np_thru_hole circle (at -7.62 5.08 180) (size 1.7 1.7) (drill 1.7) (layers "*.Cu" "*.Mask"))
  (pad "" np_thru_hole circle (at -2.54 5.08 180) (size 4 4) (drill 4) (layers "*.Cu" "*.Mask"))
  (pad "" np_thru_hole circle (at 2.54 5.08 180) (size 1.7 1.7) (drill 1.7) (layers "*.Cu" "*.Mask"))
  (pad "1" thru_hole circle (at 0 0 180) (size 2.2 2.2) (drill 1.5) (layers "*.Cu" "*.Mask") (remove_unused_layers no) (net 1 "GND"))
  (pad "2" thru_hole circle (at -6.35 2.54 180) (size 2.2 2.2) (drill 1.5) (layers "*.Cu" "*.Mask") (remove_unused_layers no) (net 3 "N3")))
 (gr_rect (start 104.775 71.4375) (end 167.265423 138.1125) (stroke (width 0.05) (type default)) (fill no) (layer "Edge.Cuts"))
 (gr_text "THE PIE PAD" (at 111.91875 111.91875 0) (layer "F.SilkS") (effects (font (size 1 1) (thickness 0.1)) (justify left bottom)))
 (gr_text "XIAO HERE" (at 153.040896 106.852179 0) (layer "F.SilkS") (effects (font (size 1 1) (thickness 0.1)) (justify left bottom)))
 (segment (start 161.76625 114.3) (end 161.76625 116.99875) (width 0.2) (layer "F.Cu") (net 1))
 (segment (start 119.22125 121.285) (end 119.04475 121.1085) (width 0.2) (layer "F.Cu") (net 1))
 (segment (start 114.14125 88.42375) (end 133.19125 88.42375) (width 0.2) (layer "F.Cu") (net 1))
 (segment (start 119.22125 121.44375) (end 119.22125 121.285) (width 0.2) (layer "F.Cu") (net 1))
 (segment (start 161.76625 116.99875) (end 157.32125 121.44375) (width 0.2) (layer "F.Cu") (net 1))
 (segment (start 109.405902 100.500525) (end 110.189475 100.500525) (width 0.2) (layer "B.Cu") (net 1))
 (segment (start 157.32125 121.44375) (end 138.27125 121.44375) (width 0.2) (layer "B.Cu") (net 1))
 (segment (start 114.14125 96.54875) (end 114.14125 88.42375) (width 0.2) (layer "B.Cu") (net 1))
 (segment (start 110.189475 100.500525) (end 114.14125 96.54875) (width 0.2) (layer "B.Cu") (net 1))
 (segment (start 143.35125 88.42375) (end 138.27125 93.50375) (width 0.2) (layer "B.Cu") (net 1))
 (segment (start 138.27125 93.50375) (end 138.27125 102.39375) (width 0.2) (layer "B.Cu") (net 1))
 (segment (start 138.27125 121.44375) (end 119.22125 121.44375) (width 0.2) (layer "B.Cu") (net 1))
 (segment (start 138.27125 121.44375) (end 138.27125 102.39375) (width 0.2) (layer "B.Cu") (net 1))
 (segment (start 133.19125 88.42375) (end 138.27125 93.50375) (width 0.2) (layer "B.Cu") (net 1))
 (segment (start 152.24125 88.42375) (end 143.35125 88.42375) (width 0.2) (layer "B.Cu") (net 1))
 (segment (start 149.06625 114.3) (end 149.06625 112.84625) (width 0.2) (layer "F.Cu") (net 9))
 (segment (start 141.15375 104.93375) (end 131.92125 104.93375) (width 0.2) (layer "F.Cu") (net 9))
 (segment (start 149.06625 112.84625) (end 141.15375 104.93375) (width 0.2) (layer "F.Cu") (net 9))
 (segment (start 151.60625 114.3) (end 151.60625 115.37763) (width 0.2) (layer "F.Cu") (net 10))
 (segment (start 118.245 118.61) (end 112.87125 123.98375) (width 0.2) (layer "F.Cu") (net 10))
 (segment (start 148.37388 118.61) (end 118.245 118.61) (width 0.2) (layer "F.Cu") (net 10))
 (segment (start 151.60625 115.37763) (end 148.37388 118.61) (width 0.2) (layer "F.Cu") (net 10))
 (segment (start 154.14625 115.37763) (end 149.76388 119.76) (width 0.2) (layer "F.Cu") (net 11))
 (segment (start 154.14625 114.3) (end 154.14625 115.37763) (width 0.2) (layer "F.Cu") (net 11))
 (segment (start 149.76388 119.76) (end 136.145 119.76) (width 0.2) (layer "F.Cu") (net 11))
 (segment (start 136.145 119.76) (end 131.92125 123.98375) (width 0.2) (layer "F.Cu") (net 11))
 (segment (start 150.97125 123.98375) (end 156.68625 118.26875) (width 0.2) (layer "F.Cu") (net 12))
 (segment (start 156.68625 118.26875) (end 156.68625 114.3) (width 0.2) (layer "F.Cu") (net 12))
 (segment (start 154.97625 100.77) (end 156.68625 99.06) (width 0.2) (layer "F.Cu") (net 5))
 (segment (start 109.405902 103.000525) (end 110.945377 104.54) (width 0.2) (layer "F.Cu") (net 5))
 (segment (start 110.945377 104.54) (end 127.89 104.54) (width 0.2) (layer "F.Cu") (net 5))
 (segment (start 131.66 100.77) (end 154.97625 100.77) (width 0.2) (layer "F.Cu") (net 5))
 (segment (start 127.89 104.54) (end 131.66 100.77) (width 0.2) (layer "F.Cu") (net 5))
 (segment (start 126.783427 100.123) (end 150.54325 100.123) (width 0.2) (layer "F.Cu") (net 7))
 (segment (start 123.905902 103.000525) (end 126.783427 100.123) (width 0.2) (layer "F.Cu") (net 7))
 (segment (start 150.54325 100.123) (end 151.60625 99.06) (width 0.2) (layer "F.Cu") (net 7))
 (segment (start 159.22625 99.06) (end 160.28925 100.123) (width 0.2) (layer "F.Cu") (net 2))
 (segment (start 162.82925 99.50031) (end 162.82925 95.61925) (width 0.2) (layer "F.Cu") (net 2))
 (segment (start 127.280634 80.65) (end 122.046884 85.88375) (width 0.2) (layer "F.Cu") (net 2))
 (segment (start 162.82925 95.61925) (end 153.08 85.87) (width 0.2) (layer "F.Cu") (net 2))
 (segment (start 146.48 85.87) (end 141.26 80.65) (width 0.2) (layer "F.Cu") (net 2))
 (segment (start 162.20656 100.123) (end 162.82925 99.50031) (width 0.2) (layer "F.Cu") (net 2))
 (segment (start 160.28925 100.123) (end 162.20656 100.123) (width 0.2) (layer "F.Cu") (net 2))
 (segment (start 153.08 85.87) (end 146.48 85.87) (width 0.2) (layer "F.Cu") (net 2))
 (segment (start 122.046884 85.88375) (end 120.49125 85.88375) (width 0.2) (layer "F.Cu") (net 2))
 (segment (start 159.22625 99.06) (end 159.22625 97.98237) (width 0.2) (layer "F.Cu") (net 2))
 (segment (start 141.26 80.65) (end 127.280634 80.65) (width 0.2) (layer "F.Cu") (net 2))
 (segment (start 161.76625 99.06) (end 161.76625 97.98237) (width 0.2) (layer "F.Cu") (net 4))
 (segment (start 161.76625 97.98237) (end 156.65263 92.86875) (width 0.2) (layer "F.Cu") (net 4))
 (segment (start 139.54125 87.15375) (end 139.54125 85.88375) (width 0.2) (layer "F.Cu") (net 4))
 (segment (start 156.65263 92.86875) (end 145.25625 92.86875) (width 0.2) (layer "F.Cu") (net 4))
 (segment (start 145.25625 92.86875) (end 139.54125 87.15375) (width 0.2) (layer "F.Cu") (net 4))
 (segment (start 164.30625 99.06) (end 164.30625 91.59875) (width 0.2) (layer "F.Cu") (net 3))
 (segment (start 164.30625 91.59875) (end 158.59125 85.88375) (width 0.2) (layer "F.Cu") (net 3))
 (segment (start 154.14625 97.47625) (end 154.14625 98.225) (width 0.2) (layer "F.Cu") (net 6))
 (segment (start 109.405902 98.000525) (end 110.946427 96.46) (width 0.2) (layer "F.Cu") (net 6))
 (segment (start 154.14625 99.06) (end 154.14625 97.98237) (width 0.2) (layer "F.Cu") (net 6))
 (segment (start 129.75875 96.46) (end 130.30875 95.91) (width 0.2) (layer "F.Cu") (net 6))
 (segment (start 130.30875 95.91) (end 152.58 95.91) (width 0.2) (layer "F.Cu") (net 6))
 (segment (start 152.58 95.91) (end 154.14625 97.47625) (width 0.2) (layer "F.Cu") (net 6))
 (segment (start 110.946427 96.46) (end 129.75875 96.46) (width 0.2) (layer "F.Cu") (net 6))
 (segment (start 123.905902 98.000525) (end 148.841775 98.000525) (width 0.2) (layer "F.Cu") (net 8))
 (segment (start 148.841775 98.000525) (end 149.06625 98.225) (width 0.2) (layer "F.Cu") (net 8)))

